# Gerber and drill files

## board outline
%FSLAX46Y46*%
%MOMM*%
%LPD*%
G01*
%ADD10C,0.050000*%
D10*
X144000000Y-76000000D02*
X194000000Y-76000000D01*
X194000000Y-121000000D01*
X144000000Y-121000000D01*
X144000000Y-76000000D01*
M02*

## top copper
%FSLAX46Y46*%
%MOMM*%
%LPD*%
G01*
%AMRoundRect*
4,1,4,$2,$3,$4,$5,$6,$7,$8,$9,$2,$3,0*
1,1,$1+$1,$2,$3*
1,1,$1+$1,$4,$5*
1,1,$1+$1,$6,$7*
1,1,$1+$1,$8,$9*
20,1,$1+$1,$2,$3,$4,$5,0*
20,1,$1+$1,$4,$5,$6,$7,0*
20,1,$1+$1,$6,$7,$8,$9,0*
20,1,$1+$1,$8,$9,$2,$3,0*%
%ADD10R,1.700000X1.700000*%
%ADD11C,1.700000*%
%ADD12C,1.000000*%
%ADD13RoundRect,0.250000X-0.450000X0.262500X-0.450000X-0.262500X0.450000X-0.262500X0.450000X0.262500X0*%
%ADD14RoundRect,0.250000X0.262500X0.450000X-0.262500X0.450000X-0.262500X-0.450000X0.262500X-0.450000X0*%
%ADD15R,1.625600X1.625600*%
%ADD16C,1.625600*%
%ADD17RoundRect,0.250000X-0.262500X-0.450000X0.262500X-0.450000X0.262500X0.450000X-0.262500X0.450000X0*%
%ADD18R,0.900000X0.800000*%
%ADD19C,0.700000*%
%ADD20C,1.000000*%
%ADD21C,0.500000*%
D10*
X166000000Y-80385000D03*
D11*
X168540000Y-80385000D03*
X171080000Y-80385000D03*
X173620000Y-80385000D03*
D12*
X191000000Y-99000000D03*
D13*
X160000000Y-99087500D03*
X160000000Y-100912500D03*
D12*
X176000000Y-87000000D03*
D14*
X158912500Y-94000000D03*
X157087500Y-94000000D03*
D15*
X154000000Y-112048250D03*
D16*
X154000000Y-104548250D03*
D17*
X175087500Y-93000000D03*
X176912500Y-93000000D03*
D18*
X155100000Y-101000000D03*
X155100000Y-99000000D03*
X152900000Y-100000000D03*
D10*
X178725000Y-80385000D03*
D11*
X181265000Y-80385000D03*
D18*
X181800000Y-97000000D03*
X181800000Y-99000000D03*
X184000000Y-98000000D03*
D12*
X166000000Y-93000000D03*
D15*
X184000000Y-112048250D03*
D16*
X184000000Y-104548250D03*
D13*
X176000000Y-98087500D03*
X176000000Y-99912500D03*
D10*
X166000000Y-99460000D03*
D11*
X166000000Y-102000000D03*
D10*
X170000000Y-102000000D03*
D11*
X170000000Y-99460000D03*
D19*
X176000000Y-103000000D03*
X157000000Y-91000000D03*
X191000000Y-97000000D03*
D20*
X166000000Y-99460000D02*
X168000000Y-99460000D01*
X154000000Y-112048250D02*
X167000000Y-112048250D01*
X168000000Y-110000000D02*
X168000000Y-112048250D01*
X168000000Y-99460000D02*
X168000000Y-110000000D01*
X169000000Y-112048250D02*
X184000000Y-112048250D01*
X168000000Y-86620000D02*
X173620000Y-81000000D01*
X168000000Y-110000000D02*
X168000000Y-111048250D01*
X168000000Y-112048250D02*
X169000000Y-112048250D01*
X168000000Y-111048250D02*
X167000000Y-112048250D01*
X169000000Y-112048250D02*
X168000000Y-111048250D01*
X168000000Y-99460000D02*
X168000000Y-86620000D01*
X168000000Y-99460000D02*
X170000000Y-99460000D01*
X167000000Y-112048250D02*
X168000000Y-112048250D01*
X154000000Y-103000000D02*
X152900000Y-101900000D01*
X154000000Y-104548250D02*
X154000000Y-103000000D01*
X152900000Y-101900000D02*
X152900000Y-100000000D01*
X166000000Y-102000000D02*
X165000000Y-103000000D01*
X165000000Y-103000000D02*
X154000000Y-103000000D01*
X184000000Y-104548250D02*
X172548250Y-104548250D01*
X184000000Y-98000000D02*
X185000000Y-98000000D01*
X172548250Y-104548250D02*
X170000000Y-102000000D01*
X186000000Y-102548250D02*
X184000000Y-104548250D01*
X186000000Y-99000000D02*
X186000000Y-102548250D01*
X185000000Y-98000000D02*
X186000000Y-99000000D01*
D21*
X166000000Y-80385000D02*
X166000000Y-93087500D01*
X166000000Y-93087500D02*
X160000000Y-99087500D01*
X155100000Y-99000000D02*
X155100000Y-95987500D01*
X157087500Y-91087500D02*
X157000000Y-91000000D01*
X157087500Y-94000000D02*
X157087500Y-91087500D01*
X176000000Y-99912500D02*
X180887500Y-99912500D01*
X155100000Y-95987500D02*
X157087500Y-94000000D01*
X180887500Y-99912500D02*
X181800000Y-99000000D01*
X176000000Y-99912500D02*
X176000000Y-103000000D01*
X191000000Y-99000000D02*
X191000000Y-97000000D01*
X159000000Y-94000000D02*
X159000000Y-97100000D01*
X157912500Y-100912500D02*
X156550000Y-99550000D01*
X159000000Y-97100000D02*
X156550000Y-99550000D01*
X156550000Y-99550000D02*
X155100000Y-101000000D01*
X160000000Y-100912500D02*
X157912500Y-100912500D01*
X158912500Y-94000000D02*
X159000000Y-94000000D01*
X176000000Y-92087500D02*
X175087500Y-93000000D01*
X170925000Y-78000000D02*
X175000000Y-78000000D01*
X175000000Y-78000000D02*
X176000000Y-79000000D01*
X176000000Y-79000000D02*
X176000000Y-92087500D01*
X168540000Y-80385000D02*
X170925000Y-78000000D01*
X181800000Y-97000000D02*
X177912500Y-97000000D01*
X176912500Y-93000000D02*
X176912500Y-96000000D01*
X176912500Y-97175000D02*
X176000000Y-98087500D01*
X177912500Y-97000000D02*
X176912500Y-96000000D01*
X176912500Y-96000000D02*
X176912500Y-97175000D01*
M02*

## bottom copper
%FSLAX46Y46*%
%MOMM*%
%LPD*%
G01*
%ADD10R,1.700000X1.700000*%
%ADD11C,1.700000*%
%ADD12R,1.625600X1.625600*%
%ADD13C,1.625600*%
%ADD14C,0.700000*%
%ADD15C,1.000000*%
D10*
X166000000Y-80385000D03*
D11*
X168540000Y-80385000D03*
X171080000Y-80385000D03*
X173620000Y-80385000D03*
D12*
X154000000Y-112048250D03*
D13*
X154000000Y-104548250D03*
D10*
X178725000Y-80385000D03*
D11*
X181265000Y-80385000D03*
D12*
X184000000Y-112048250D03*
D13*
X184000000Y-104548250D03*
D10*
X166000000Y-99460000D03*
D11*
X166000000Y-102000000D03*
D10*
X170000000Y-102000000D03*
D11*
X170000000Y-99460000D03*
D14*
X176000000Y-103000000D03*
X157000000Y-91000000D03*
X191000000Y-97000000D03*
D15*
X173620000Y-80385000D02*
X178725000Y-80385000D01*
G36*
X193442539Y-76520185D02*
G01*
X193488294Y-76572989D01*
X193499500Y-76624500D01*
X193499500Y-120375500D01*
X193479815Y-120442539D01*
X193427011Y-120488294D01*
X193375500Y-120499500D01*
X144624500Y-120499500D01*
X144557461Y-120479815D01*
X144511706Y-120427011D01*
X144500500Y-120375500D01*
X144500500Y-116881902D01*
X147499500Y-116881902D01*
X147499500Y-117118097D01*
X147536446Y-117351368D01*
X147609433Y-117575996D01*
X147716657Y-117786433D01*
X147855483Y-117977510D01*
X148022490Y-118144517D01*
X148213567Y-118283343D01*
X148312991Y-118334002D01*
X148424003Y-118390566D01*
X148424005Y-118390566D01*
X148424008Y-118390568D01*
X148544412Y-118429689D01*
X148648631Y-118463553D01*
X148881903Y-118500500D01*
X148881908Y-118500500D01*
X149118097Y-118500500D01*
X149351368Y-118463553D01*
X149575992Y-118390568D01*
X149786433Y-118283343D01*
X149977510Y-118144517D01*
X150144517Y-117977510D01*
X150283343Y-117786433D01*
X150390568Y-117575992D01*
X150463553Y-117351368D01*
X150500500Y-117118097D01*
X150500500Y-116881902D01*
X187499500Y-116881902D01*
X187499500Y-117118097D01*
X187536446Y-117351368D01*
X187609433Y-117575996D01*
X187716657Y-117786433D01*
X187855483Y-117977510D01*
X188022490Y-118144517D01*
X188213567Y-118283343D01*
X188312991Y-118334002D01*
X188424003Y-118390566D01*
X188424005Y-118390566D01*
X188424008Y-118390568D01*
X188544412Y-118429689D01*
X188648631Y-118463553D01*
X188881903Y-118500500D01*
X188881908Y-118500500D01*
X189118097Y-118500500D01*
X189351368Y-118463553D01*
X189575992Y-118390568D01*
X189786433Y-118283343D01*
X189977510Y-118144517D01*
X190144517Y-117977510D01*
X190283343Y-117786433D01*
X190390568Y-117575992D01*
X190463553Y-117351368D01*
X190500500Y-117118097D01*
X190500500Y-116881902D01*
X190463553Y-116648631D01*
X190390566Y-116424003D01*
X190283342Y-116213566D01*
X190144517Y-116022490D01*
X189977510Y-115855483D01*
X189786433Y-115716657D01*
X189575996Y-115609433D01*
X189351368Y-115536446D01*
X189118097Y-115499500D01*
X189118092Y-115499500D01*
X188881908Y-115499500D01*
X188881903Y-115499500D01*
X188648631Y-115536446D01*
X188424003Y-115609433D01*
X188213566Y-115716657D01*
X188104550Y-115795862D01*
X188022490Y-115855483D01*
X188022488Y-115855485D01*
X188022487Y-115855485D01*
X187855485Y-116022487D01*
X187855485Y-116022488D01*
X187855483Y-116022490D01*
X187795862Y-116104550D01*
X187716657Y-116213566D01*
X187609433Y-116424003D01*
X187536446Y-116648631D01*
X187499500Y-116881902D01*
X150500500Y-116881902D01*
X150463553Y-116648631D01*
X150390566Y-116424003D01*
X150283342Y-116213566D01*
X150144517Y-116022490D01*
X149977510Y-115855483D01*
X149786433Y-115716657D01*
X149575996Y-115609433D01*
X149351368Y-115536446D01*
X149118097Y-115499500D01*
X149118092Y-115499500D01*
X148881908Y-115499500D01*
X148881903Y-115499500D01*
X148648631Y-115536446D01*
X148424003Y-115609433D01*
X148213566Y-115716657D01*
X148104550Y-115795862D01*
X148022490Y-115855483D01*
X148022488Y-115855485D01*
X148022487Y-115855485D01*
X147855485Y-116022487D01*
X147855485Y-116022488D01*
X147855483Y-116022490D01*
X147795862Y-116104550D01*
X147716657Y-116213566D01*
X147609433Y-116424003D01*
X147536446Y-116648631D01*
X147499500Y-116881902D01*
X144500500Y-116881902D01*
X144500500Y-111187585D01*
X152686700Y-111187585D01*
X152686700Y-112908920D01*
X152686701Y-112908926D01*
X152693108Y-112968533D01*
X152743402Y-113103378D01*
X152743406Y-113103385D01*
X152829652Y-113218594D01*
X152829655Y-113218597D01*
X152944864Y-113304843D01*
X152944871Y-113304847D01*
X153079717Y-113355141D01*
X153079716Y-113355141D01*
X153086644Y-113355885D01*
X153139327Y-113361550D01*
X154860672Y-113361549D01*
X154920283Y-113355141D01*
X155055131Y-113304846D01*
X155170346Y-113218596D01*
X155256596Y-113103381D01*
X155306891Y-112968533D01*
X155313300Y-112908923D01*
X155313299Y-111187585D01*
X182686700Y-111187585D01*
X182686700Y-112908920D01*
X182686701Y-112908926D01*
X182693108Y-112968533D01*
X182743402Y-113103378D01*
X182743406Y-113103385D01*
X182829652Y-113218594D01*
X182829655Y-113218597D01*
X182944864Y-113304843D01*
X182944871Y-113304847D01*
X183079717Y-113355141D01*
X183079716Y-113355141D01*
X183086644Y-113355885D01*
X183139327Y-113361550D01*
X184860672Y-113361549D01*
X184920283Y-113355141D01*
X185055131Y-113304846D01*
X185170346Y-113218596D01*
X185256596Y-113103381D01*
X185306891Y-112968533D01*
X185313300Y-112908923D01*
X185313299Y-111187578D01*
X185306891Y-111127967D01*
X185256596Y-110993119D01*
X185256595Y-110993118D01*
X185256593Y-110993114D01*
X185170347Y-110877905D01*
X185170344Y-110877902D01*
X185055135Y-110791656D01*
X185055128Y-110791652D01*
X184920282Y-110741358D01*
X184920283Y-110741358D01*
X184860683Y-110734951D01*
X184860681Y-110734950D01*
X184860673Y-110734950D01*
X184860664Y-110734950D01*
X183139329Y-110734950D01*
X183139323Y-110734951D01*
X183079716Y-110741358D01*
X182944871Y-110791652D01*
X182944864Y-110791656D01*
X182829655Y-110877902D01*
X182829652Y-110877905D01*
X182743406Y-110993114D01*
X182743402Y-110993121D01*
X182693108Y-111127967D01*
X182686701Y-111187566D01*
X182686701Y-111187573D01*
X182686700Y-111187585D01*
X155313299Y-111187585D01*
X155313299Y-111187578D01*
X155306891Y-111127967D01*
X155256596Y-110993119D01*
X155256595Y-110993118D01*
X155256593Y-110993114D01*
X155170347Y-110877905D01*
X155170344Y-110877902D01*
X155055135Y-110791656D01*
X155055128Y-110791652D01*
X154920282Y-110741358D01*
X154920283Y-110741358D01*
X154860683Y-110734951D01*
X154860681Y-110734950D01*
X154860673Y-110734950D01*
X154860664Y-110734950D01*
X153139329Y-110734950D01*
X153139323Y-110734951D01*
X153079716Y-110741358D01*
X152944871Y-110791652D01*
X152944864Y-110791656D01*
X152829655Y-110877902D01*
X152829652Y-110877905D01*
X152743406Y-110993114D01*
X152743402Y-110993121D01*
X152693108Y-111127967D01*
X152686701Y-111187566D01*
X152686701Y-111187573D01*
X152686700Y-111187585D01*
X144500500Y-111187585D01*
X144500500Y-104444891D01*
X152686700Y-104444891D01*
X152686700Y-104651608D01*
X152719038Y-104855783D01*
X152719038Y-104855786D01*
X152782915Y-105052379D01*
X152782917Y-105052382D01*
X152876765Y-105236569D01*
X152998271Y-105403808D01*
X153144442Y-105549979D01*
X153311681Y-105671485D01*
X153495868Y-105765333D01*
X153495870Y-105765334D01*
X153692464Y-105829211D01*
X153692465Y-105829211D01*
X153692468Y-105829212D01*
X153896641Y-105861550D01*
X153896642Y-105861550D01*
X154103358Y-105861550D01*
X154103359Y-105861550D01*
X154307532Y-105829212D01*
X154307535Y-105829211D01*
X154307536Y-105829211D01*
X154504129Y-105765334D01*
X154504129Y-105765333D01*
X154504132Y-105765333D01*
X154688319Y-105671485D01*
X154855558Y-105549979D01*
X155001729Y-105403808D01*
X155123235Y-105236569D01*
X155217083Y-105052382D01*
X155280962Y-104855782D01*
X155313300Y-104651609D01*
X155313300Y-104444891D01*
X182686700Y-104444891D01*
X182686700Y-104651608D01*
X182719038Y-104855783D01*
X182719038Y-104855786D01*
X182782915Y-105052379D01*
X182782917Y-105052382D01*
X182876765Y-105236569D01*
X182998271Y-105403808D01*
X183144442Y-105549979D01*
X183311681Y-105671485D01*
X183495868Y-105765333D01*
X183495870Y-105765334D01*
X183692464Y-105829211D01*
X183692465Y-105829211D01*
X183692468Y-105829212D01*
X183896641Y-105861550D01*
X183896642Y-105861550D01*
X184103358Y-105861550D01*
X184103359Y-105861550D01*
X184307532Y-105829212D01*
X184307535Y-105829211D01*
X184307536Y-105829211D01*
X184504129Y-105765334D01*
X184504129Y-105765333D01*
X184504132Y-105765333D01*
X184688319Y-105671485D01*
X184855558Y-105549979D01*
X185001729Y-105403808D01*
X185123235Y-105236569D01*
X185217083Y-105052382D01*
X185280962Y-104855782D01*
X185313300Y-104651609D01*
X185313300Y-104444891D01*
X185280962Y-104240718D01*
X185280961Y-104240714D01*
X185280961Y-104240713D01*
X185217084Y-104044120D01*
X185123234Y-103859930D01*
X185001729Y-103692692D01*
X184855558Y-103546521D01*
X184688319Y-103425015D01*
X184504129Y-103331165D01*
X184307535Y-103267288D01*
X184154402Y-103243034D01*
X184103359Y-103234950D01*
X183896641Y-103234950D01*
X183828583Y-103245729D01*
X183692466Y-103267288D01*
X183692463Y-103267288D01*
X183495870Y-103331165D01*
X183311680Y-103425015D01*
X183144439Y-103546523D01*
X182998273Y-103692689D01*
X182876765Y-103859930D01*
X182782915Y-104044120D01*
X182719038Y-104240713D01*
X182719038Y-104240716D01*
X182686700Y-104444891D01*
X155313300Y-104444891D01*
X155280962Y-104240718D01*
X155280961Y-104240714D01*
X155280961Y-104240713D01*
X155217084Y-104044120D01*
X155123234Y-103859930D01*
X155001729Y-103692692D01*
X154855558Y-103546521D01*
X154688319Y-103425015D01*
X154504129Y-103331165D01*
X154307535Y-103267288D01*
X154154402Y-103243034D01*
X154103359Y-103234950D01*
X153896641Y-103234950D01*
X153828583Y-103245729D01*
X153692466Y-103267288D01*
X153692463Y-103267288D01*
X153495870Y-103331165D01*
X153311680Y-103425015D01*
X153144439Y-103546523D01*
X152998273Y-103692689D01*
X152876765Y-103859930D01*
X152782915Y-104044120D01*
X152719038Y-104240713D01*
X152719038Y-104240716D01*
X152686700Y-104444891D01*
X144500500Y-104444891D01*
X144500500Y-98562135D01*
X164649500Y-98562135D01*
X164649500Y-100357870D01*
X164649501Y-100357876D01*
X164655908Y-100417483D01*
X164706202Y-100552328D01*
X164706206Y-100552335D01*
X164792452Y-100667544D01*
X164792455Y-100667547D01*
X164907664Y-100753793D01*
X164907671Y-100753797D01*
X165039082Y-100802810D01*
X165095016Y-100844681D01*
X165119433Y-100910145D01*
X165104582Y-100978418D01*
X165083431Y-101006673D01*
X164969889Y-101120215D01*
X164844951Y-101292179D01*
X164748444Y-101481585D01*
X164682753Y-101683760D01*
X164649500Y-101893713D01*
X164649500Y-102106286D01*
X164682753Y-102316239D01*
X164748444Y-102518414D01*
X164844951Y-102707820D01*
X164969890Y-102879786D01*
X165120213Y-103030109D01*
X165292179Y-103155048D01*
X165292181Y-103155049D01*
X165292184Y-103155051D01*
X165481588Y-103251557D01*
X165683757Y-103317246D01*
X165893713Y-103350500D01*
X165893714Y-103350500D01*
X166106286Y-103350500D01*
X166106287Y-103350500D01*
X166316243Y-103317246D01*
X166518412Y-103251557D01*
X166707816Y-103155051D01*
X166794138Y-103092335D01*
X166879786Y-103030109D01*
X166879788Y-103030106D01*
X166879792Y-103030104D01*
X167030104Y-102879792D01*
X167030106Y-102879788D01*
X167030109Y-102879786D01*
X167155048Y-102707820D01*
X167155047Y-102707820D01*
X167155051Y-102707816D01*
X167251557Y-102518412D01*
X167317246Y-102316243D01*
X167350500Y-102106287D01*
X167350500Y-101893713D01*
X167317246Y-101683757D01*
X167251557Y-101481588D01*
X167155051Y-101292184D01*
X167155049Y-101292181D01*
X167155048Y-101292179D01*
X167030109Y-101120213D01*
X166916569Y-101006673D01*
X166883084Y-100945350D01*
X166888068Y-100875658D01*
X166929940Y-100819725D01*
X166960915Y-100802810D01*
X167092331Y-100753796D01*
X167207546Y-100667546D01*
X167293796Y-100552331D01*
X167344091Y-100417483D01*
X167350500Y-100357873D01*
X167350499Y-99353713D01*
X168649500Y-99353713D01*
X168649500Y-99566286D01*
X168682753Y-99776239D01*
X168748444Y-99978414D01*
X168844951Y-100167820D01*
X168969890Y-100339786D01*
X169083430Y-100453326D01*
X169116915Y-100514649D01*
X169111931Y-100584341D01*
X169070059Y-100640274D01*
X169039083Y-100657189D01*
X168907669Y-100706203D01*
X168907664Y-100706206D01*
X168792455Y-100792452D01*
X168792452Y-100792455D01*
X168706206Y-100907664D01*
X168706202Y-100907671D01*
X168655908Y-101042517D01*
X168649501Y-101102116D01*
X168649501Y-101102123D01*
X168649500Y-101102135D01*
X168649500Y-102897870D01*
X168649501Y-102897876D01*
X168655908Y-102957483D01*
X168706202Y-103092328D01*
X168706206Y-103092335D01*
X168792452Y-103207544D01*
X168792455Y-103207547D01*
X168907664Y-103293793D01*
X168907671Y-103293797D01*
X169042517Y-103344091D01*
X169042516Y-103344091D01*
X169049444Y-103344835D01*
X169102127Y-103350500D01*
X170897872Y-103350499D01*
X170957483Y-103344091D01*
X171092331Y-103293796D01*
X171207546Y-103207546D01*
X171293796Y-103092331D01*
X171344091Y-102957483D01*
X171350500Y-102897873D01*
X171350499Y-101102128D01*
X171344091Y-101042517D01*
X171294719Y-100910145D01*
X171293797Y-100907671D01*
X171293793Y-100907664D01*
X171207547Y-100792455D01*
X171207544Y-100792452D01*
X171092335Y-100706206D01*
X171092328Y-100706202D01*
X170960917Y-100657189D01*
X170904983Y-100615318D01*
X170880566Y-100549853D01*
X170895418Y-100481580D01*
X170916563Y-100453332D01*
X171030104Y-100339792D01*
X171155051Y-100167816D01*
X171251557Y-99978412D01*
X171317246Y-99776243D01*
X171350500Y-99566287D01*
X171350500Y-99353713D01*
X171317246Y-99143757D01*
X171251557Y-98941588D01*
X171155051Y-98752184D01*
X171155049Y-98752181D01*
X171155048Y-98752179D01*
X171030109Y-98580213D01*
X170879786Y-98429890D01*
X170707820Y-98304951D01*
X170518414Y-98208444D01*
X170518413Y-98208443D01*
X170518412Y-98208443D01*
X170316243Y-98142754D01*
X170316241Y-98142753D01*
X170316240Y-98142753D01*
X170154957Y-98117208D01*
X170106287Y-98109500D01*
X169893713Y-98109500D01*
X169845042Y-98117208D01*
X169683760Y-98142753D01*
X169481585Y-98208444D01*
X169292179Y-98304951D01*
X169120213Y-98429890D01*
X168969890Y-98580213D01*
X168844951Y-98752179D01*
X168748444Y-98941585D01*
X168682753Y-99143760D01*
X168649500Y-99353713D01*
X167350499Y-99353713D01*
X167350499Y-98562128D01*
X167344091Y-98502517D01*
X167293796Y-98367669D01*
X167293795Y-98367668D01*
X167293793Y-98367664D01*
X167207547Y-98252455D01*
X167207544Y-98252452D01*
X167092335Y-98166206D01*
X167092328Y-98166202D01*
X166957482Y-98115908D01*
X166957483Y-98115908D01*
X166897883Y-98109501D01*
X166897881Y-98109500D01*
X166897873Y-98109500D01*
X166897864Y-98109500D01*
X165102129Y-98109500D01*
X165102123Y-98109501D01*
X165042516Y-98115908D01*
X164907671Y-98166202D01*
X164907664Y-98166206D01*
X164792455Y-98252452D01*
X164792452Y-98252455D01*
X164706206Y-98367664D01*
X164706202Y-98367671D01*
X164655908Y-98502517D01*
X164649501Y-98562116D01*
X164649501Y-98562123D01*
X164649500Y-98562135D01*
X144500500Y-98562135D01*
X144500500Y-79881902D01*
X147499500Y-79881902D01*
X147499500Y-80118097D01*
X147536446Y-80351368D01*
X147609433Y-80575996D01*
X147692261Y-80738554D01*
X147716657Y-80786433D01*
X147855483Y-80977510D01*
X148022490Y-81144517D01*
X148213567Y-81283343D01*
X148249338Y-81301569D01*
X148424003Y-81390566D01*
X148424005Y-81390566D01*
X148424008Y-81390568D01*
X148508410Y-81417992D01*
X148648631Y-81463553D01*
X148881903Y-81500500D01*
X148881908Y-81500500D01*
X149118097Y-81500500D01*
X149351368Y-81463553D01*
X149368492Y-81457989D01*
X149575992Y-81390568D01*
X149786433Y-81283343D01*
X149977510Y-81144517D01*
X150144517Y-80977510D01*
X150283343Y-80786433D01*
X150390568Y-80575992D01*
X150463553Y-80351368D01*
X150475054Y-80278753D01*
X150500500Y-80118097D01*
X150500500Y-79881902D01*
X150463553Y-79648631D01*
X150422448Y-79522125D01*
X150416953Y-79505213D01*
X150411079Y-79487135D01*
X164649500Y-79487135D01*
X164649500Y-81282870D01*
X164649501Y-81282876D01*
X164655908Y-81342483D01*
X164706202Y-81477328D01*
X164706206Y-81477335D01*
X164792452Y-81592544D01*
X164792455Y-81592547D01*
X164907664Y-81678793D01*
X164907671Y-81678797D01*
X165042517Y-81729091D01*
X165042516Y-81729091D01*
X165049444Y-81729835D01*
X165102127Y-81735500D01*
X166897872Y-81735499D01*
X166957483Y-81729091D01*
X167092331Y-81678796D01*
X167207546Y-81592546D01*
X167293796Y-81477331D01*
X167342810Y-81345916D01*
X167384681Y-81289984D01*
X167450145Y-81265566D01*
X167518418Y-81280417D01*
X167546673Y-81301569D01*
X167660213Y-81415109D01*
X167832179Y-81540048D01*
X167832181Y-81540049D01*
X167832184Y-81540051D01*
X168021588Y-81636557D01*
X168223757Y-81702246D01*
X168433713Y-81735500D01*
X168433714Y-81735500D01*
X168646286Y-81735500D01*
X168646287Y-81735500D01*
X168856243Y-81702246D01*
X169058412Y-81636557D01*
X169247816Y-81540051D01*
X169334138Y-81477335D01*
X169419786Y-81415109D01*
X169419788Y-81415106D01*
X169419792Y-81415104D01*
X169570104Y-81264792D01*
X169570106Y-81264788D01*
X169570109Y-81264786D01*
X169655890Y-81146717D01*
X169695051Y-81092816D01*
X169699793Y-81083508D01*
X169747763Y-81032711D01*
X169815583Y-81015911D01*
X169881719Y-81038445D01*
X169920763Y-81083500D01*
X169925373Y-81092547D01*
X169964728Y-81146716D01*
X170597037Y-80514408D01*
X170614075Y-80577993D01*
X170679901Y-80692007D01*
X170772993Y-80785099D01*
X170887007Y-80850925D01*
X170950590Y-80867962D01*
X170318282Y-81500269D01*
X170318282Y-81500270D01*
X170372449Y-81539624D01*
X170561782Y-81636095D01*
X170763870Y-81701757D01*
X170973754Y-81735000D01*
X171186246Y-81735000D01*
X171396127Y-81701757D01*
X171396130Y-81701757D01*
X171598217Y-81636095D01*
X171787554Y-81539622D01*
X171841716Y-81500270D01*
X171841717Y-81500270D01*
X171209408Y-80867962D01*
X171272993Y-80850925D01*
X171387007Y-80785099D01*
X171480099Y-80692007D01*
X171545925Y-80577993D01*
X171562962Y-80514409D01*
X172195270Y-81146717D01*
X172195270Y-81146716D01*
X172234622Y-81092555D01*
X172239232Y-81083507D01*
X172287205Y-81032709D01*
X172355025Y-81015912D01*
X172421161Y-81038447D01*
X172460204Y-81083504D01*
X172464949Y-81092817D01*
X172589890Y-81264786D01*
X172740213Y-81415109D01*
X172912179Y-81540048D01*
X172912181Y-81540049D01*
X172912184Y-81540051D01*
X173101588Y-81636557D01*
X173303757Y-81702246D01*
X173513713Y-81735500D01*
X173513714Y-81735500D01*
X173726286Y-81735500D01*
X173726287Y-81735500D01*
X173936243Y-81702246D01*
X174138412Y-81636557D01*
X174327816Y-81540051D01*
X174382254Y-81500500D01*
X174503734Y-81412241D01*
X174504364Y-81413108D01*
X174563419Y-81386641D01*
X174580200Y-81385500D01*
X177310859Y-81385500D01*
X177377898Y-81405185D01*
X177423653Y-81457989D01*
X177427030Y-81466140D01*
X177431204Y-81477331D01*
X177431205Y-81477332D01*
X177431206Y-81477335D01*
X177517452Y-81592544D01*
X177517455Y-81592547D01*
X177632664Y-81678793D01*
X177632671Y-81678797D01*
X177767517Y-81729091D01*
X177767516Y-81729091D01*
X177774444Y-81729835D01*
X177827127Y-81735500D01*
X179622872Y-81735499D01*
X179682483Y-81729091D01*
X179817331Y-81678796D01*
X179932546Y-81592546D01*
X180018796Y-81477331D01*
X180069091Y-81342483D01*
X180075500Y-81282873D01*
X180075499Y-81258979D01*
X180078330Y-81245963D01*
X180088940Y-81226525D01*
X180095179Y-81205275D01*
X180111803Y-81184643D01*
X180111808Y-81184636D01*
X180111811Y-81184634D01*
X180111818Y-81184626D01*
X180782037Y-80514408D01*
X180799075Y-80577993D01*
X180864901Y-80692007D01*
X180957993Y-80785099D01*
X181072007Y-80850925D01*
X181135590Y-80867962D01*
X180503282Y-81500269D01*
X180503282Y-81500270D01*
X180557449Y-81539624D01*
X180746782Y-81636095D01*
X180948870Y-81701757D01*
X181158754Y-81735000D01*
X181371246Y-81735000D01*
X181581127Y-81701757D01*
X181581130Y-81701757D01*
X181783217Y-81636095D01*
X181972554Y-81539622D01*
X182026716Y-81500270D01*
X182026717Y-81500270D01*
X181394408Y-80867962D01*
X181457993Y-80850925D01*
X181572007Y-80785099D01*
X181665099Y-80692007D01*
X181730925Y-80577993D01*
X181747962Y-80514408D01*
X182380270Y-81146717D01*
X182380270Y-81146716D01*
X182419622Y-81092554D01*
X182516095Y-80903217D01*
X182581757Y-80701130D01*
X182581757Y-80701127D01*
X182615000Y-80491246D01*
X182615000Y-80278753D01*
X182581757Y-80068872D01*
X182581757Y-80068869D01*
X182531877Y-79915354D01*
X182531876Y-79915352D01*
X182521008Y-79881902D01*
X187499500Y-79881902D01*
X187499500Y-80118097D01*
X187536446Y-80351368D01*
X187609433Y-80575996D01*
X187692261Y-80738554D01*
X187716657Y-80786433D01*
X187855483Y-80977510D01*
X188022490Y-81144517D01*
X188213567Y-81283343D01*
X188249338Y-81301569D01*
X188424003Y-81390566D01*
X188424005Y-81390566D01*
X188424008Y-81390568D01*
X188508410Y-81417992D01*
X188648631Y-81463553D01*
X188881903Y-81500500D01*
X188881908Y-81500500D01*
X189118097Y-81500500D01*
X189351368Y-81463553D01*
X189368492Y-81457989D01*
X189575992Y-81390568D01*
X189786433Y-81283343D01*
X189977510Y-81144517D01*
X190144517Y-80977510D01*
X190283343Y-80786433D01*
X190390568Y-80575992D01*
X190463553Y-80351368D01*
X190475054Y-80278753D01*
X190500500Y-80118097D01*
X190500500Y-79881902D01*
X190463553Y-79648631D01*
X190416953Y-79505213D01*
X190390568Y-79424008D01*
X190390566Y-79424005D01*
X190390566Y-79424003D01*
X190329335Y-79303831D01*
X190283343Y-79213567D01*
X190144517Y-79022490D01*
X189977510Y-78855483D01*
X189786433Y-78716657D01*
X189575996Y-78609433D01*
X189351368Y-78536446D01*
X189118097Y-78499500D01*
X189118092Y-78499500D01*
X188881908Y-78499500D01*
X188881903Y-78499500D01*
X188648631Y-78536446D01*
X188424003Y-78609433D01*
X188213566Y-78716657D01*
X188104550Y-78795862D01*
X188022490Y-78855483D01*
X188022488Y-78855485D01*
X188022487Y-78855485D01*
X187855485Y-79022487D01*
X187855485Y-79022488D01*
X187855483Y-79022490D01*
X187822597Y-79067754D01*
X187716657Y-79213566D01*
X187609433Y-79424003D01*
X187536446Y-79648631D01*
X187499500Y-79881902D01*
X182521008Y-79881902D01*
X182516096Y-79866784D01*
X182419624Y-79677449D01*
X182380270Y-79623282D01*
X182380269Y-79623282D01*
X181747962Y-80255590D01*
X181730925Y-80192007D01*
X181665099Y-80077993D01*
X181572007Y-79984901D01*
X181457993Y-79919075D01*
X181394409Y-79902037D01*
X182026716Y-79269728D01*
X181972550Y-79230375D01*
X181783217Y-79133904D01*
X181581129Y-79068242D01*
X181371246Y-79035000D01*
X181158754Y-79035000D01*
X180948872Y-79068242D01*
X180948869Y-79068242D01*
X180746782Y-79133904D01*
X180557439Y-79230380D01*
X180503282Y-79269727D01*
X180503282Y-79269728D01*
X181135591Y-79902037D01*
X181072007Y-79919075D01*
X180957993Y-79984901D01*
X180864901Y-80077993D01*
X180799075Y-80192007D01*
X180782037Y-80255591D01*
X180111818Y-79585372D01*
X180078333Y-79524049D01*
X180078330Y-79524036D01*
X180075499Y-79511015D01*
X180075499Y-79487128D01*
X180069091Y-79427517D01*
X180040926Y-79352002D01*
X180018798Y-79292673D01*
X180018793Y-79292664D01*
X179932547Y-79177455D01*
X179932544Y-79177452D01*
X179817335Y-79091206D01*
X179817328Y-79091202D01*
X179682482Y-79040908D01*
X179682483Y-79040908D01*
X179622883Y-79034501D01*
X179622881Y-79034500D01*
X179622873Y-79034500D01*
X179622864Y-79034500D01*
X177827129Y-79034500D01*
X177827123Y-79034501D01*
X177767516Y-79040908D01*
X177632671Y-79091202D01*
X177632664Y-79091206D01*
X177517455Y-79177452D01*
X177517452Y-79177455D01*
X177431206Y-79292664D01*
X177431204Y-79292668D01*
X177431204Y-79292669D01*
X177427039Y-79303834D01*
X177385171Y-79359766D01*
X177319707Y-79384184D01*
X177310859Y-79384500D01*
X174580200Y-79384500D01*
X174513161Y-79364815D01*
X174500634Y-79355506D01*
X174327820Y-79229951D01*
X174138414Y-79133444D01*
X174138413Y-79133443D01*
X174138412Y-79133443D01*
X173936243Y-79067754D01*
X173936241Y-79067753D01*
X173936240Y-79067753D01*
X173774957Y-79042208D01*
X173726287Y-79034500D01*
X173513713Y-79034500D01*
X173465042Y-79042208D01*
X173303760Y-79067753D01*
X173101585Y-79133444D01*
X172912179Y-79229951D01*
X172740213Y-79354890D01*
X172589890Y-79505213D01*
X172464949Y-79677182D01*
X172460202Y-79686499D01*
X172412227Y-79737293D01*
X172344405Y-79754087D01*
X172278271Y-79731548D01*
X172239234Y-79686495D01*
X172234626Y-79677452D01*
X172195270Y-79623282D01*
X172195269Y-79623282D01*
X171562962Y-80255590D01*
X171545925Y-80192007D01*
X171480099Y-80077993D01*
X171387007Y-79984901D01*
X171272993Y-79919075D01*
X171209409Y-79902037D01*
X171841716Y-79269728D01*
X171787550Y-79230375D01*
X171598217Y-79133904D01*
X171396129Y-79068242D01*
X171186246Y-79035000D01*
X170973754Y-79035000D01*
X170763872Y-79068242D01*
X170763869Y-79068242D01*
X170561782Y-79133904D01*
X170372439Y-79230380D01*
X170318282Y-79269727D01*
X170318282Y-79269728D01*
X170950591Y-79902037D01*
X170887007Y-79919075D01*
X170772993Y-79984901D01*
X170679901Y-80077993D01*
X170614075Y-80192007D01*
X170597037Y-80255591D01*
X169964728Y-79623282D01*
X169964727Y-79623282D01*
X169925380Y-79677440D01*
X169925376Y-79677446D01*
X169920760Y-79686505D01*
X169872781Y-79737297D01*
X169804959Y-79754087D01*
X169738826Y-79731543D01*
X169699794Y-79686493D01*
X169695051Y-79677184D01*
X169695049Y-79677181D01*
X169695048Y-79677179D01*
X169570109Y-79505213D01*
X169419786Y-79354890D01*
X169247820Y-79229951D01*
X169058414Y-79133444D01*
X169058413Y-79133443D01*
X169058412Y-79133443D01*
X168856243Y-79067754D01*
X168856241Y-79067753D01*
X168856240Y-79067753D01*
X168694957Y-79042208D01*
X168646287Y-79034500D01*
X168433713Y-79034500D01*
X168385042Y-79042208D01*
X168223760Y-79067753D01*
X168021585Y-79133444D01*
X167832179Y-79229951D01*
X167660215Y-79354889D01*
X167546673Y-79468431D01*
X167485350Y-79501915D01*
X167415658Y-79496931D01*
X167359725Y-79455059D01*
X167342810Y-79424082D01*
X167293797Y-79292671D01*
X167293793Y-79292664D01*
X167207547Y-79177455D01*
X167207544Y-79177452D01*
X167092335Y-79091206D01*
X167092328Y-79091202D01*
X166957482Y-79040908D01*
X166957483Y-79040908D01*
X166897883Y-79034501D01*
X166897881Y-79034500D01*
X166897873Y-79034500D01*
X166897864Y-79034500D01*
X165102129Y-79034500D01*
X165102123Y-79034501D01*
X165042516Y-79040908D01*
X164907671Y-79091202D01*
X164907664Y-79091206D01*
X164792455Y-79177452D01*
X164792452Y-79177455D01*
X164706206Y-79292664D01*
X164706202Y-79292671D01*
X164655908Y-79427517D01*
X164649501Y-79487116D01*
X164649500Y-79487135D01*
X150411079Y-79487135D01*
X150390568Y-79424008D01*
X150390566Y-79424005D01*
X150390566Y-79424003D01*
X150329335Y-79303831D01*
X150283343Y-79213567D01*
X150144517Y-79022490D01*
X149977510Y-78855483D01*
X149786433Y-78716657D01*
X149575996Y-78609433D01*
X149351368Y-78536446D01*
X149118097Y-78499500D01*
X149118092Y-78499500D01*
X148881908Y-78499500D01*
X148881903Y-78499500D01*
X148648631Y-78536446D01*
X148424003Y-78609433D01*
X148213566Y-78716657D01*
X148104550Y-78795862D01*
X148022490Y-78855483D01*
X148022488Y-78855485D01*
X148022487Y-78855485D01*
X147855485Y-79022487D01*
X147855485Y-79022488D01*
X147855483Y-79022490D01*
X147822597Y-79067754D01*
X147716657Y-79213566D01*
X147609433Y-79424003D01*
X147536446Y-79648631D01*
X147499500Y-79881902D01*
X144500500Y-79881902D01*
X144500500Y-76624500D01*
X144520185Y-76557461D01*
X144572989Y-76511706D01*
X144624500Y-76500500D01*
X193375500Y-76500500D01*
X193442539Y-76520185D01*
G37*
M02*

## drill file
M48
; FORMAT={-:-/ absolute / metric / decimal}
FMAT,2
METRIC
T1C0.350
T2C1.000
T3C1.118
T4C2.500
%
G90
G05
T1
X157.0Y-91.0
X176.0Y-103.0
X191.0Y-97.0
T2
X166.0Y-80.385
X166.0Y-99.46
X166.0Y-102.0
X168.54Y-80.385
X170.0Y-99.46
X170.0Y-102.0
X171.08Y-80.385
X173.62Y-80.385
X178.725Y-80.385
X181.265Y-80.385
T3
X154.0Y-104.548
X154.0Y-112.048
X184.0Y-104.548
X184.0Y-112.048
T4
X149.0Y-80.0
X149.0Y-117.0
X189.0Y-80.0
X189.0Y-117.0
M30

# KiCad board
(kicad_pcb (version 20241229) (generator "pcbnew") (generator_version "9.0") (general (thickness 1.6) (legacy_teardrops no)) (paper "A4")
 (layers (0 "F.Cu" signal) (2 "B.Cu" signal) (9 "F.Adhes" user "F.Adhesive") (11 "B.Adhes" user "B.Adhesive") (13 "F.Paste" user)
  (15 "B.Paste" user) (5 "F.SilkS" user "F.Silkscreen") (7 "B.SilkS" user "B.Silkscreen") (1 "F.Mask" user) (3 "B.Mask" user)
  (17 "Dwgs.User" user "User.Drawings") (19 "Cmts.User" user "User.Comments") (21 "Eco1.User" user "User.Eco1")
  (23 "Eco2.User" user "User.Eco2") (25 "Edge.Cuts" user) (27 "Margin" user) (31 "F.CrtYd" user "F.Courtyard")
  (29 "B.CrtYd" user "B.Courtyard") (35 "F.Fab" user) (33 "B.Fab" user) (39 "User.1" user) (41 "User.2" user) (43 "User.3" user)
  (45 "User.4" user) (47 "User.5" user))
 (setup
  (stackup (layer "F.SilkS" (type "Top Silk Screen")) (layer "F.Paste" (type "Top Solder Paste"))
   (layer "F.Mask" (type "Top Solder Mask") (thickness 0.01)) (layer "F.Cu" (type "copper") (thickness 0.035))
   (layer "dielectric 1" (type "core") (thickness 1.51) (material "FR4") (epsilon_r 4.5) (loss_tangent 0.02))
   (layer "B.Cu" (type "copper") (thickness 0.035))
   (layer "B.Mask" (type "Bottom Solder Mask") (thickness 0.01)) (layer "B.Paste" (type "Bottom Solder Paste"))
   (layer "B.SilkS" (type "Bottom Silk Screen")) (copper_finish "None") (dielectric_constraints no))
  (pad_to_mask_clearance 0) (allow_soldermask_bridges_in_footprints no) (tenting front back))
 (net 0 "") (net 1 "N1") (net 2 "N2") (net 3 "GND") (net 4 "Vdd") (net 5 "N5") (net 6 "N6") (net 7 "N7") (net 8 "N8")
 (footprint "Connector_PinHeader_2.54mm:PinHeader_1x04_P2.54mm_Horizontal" (layer "F.Cu") (at 166 80.385 90)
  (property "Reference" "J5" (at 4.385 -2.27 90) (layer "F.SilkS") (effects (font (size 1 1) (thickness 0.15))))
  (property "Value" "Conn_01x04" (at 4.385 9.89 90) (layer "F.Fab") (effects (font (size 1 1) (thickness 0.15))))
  (pad "1" thru_hole rect (at 0 0 90) (size 1.7 1.7) (drill 1) (layers "*.Cu" "*.Mask") (remove_unused_layers no) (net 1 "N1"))
  (pad "2" thru_hole circle (at 0 2.54 90) (size 1.7 1.7) (drill 1) (layers "*.Cu" "*.Mask") (remove_unused_layers no) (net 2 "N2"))
  (pad "3" thru_hole circle (at 0 5.08 90) (size 1.7 1.7) (drill 1) (layers "*.Cu" "*.Mask") (remove_unused_layers no) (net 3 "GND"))
  (pad "4" thru_hole circle (at 0 7.62 90) (size 1.7 1.7) (drill 1) (layers "*.Cu" "*.Mask") (remove_unused_layers no) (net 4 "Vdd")))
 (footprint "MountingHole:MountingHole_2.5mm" (layer "F.Cu") (at 189 80)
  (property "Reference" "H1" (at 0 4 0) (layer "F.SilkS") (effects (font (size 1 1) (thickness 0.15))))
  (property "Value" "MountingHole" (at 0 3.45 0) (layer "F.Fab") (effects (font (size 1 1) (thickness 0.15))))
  (pad "" np_thru_hole circle (at 0 0) (size 2.5 2.5) (drill 2.5) (layers "*.Cu" "*.Mask")))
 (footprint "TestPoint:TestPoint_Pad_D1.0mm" (layer "F.Cu") (at 191 99)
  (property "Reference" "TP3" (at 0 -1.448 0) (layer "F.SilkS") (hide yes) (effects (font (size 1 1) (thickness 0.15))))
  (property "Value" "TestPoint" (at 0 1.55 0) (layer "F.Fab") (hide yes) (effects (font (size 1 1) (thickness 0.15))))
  (pad "1" smd circle (at 0 0) (size 1 1) (layers "F.Cu" "F.Mask") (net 3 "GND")))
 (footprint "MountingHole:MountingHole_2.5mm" (layer "F.Cu") (at 189 117)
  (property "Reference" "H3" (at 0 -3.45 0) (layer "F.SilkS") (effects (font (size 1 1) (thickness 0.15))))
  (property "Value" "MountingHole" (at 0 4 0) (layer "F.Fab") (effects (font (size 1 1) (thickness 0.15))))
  (pad "" np_thru_hole circle (at 0 0) (size 2.5 2.5) (drill 2.5) (layers "*.Cu" "*.Mask")))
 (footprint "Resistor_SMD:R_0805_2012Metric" (layer "F.Cu") (at 160 100 -90)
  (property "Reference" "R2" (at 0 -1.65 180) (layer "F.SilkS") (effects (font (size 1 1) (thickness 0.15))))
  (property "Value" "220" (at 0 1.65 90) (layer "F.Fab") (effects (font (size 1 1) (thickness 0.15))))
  (pad "1" smd roundrect (at -0.9125 0 270) (size 1.025 1.4) (layers "F.Cu" "F.Mask" "F.Paste") (roundrect_rratio 0.243902) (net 1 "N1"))
  (pad "2" smd roundrect (at 0.9125 0 270) (size 1.025 1.4) (layers "F.Cu" "F.Mask" "F.Paste") (roundrect_rratio 0.243902) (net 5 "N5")))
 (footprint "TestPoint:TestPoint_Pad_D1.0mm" (layer "F.Cu") (at 176 87)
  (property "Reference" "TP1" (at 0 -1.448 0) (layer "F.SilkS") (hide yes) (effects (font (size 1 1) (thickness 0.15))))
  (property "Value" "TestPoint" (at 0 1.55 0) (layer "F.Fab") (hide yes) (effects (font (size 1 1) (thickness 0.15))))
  (pad "1" smd circle (at 0 0) (size 1 1) (layers "F.Cu" "F.Mask") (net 2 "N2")))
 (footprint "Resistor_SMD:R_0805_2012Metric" (layer "F.Cu") (at 158 94 180)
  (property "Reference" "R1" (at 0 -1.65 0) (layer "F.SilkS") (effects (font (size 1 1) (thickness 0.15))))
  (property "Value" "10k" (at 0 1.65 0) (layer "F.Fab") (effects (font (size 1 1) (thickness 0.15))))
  (pad "1" smd roundrect (at -0.9125 0 180) (size 1.025 1.4) (layers "F.Cu" "F.Mask" "F.Paste") (roundrect_rratio 0.243902) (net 5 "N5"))
  (pad "2" smd roundrect (at 0.9125 0 180) (size 1.025 1.4) (layers "F.Cu" "F.Mask" "F.Paste") (roundrect_rratio 0.243902) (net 3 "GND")))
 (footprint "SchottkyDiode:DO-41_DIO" (layer "F.Cu") (at 154 114.04825 90)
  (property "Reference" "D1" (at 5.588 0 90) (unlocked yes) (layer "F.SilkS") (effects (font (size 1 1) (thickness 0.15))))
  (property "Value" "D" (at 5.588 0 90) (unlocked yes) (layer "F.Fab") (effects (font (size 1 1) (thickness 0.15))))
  (pad "1" thru_hole rect (at 2 0 90) (size 1.6256 1.6256) (drill 1.1176) (layers "*.Cu" "*.Mask") (remove_unused_layers no) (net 4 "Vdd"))
  (pad "2" thru_hole circle (at 9.5 0 90) (size 1.6256 1.6256) (drill 1.1176) (layers "*.Cu" "*.Mask") (remove_unused_layers no)
   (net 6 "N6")))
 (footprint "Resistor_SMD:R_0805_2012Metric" (layer "F.Cu") (at 176 93)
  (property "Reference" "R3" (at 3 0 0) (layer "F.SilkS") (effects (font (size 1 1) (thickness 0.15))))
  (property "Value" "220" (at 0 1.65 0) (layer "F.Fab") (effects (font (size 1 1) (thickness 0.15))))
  (pad "1" smd roundrect (at -0.9125 0) (size 1.025 1.4) (layers "F.Cu" "F.Mask" "F.Paste") (roundrect_rratio 0.243902) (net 2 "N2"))
  (pad "2" smd roundrect (at 0.9125 0) (size 1.025 1.4) (layers "F.Cu" "F.Mask" "F.Paste") (roundrect_rratio 0.243902) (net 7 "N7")))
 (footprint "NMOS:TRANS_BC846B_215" (layer "F.Cu") (at 154 100 90)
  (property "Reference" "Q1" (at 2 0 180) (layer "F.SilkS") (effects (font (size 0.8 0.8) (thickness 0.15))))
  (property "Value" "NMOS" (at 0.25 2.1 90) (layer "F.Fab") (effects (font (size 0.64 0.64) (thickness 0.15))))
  (pad "1" smd rect (at -1 1.1 90) (size 0.8 0.9) (layers "F.Cu" "F.Mask" "F.Paste") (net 5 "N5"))
  (pad "2" smd rect (at 1 1.1 90) (size 0.8 0.9) (layers "F.Cu" "F.Mask" "F.Paste") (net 3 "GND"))
  (pad "3" smd rect (at 0 -1.1 90) (size 0.8 0.9) (layers "F.Cu" "F.Mask" "F.Paste") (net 6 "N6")))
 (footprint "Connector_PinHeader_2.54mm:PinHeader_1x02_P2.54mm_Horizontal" (layer "F.Cu") (at 178.725 80.385 90)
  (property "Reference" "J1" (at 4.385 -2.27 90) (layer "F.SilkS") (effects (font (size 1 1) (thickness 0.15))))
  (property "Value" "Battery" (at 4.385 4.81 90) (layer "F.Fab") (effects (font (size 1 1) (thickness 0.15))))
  (pad "1" thru_hole rect (at 0 0 90) (size 1.7 1.7) (drill 1) (layers "*.Cu" "*.Mask") (remove_unused_layers no) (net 4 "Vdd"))
  (pad "2" thru_hole circle (at 0 2.54 90) (size 1.7 1.7) (drill 1) (layers "*.Cu" "*.Mask") (remove_unused_layers no) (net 3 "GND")))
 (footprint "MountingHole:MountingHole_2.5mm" (layer "F.Cu") (at 149 80)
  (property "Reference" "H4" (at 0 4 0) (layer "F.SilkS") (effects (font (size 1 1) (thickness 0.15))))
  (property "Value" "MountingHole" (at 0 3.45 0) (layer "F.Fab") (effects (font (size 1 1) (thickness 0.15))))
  (pad "" np_thru_hole circle (at 0 0) (size 2.5 2.5) (drill 2.5) (layers "*.Cu" "*.Mask")))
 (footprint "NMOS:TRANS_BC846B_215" (layer "F.Cu") (at 182.9 98 -90)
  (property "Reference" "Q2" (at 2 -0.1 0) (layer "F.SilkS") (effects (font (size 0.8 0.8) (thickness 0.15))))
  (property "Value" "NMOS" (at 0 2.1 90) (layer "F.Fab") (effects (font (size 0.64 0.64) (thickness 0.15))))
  (pad "1" smd rect (at -1 1.1 270) (size 0.8 0.9) (layers "F.Cu" "F.Mask" "F.Paste") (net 7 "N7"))
  (pad "2" smd rect (at 1 1.1 270) (size 0.8 0.9) (layers "F.Cu" "F.Mask" "F.Paste") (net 3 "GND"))
  (pad "3" smd rect (at 0 -1.1 270) (size 0.8 0.9) (layers "F.Cu" "F.Mask" "F.Paste") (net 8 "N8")))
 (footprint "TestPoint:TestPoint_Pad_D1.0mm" (layer "F.Cu") (at 166 93)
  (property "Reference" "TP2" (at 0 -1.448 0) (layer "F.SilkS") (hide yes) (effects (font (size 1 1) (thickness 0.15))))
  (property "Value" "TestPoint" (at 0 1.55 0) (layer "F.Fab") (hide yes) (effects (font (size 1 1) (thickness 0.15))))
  (pad "1" smd circle (at 0 0) (size 1 1) (layers "F.Cu" "F.Mask") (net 1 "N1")))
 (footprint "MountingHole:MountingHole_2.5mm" (layer "F.Cu") (at 149 117)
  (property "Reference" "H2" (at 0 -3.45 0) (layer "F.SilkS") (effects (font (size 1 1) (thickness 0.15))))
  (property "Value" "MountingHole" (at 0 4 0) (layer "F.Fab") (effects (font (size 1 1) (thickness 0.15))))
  (pad "" np_thru_hole circle (at 0 0) (size 2.5 2.5) (drill 2.5) (layers "*.Cu" "*.Mask")))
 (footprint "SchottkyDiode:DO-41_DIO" (layer "F.Cu") (at 184 114.04825 90)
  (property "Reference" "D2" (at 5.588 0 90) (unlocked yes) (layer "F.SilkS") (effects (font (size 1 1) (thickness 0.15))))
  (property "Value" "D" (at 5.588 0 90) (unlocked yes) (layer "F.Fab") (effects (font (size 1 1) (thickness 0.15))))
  (pad "1" thru_hole rect (at 2 0 90) (size 1.6256 1.6256) (drill 1.1176) (layers "*.Cu" "*.Mask") (remove_unused_layers no) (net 4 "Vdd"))
  (pad "2" thru_hole circle (at 9.5 0 90) (size 1.6256 1.6256) (drill 1.1176) (layers "*.Cu" "*.Mask") (remove_unused_layers no)
   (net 8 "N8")))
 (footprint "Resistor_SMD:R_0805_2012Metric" (layer "F.Cu") (at 176 99 -90)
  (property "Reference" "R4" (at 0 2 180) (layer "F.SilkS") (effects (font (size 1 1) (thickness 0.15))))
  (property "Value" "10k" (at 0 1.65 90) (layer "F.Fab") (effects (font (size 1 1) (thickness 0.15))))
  (pad "1" smd roundrect (at -0.9125 0 270) (size 1.025 1.4) (layers "F.Cu" "F.Mask" "F.Paste") (roundrect_rratio 0.243902) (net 7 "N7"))
  (pad "2" smd roundrect (at 0.9125 0 270) (size 1.025 1.4) (layers "F.Cu" "F.Mask" "F.Paste") (roundrect_rratio 0.243902) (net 3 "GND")))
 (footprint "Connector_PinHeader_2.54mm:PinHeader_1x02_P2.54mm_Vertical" (layer "B.Cu") (at 166 99.46 180)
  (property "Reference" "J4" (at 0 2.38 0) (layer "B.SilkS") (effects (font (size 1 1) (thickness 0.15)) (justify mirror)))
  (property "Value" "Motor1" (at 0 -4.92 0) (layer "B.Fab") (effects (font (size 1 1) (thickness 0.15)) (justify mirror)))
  (pad "1" thru_hole rect (at 0 0 180) (size 1.7 1.7) (drill 1) (layers "*.Cu" "*.Mask") (remove_unused_layers no) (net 4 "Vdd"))
  (pad "2" thru_hole circle (at 0 -2.54 180) (size 1.7 1.7) (drill 1) (layers "*.Cu" "*.Mask") (remove_unused_layers no) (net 6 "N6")))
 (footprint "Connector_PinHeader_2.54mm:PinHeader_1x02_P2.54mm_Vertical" (layer "B.Cu") (at 170 102)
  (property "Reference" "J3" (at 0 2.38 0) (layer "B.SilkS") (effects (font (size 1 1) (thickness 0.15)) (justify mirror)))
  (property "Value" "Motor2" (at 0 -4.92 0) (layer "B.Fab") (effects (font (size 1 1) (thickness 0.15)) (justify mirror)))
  (pad "1" thru_hole rect (at 0 0) (size 1.7 1.7) (drill 1) (layers "*.Cu" "*.Mask") (remove_unused_layers no) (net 8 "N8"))
  (pad "2" thru_hole circle (at 0 -2.54) (size 1.7 1.7) (drill 1) (layers "*.Cu" "*.Mask") (remove_unused_layers no) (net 4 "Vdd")))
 (gr_rect (start 144 76) (end 194 121) (stroke (width 0.05) (type default)) (fill no) (layer "Edge.Cuts"))
 (segment (start 166 99.46) (end 168 99.46) (width 1) (layer "F.Cu") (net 4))
 (segment (start 154 112.04825) (end 167 112.04825) (width 1) (layer "F.Cu") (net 4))
 (segment (start 168 110) (end 168 112.04825) (width 1) (layer "F.Cu") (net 4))
 (segment (start 168 99.46) (end 168 110) (width 1) (layer "F.Cu") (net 4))
 (segment (start 169 112.04825) (end 184 112.04825) (width 1) (layer "F.Cu") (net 4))
 (segment (start 168 86.62) (end 173.62 81) (width 1) (layer "F.Cu") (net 4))
 (segment (start 168 110) (end 168 111.04825) (width 1) (layer "F.Cu") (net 4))
 (segment (start 168 112.04825) (end 169 112.04825) (width 1) (layer "F.Cu") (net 4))
 (segment (start 168 111.04825) (end 167 112.04825) (width 1) (layer "F.Cu") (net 4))
 (segment (start 169 112.04825) (end 168 111.04825) (width 1) (layer "F.Cu") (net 4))
 (segment (start 168 99.46) (end 168 86.62) (width 1) (layer "F.Cu") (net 4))
 (segment (start 168 99.46) (end 170 99.46) (width 1) (layer "F.Cu") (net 4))
 (segment (start 167 112.04825) (end 168 112.04825) (width 1) (layer "F.Cu") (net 4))
 (segment (start 173.62 80.385) (end 178.725 80.385) (width 1) (layer "B.Cu") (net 4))
 (segment (start 154 103) (end 152.9 101.9) (width 1) (layer "F.Cu") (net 6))
 (segment (start 154 104.54825) (end 154 103) (width 1) (layer "F.Cu") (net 6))
 (segment (start 152.9 101.9) (end 152.9 100) (width 1) (layer "F.Cu") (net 6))
 (segment (start 166 102) (end 165 103) (width 1) (layer "F.Cu") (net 6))
 (segment (start 165 103) (end 154 103) (width 1) (layer "F.Cu") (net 6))
 (segment (start 184 104.54825) (end 172.54825 104.54825) (width 1) (layer "F.Cu") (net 8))
 (segment (start 184 98) (end 185 98) (width 1) (layer "F.Cu") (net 8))
 (segment (start 172.54825 104.54825) (end 170 102) (width 1) (layer "F.Cu") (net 8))
 (segment (start 186 102.54825) (end 184 104.54825) (width 1) (layer "F.Cu") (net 8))
 (segment (start 186 99) (end 186 102.54825) (width 1) (layer "F.Cu") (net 8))
 (segment (start 185 98) (end 186 99) (width 1) (layer "F.Cu") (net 8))
 (segment (start 166 80.385) (end 166 93.0875) (width 0.5) (layer "F.Cu") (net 1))
 (segment (start 166 93.0875) (end 160 99.0875) (width 0.5) (layer "F.Cu") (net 1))
 (segment (start 155.1 99) (end 155.1 95.9875) (width 0.5) (layer "F.Cu") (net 3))
 (segment (start 157.0875 91.0875) (end 157 91) (width 0.5) (layer "F.Cu") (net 3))
 (segment (start 157.0875 94) (end 157.0875 91.0875) (width 0.5) (layer "F.Cu") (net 3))
 (segment (start 176 99.9125) (end 180.8875 99.9125) (width 0.5) (layer "F.Cu") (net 3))
 (segment (start 155.1 95.9875) (end 157.0875 94) (width 0.5) (layer "F.Cu") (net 3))
 (segment (start 180.8875 99.9125) (end 181.8 99) (width 0.5) (layer "F.Cu") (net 3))
 (segment (start 176 99.9125) (end 176 103) (width 0.5) (layer "F.Cu") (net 3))
 (segment (start 191 99) (end 191 97) (width 0.5) (layer "F.Cu") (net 3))
 (via (at 176 103) (size 0.7) (drill 0.35) (layers "F.Cu" "B.Cu") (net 3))
 (via (at 157 91) (size 0.7) (drill 0.35) (layers "F.Cu" "B.Cu") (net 3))
 (via (at 191 97) (size 0.7) (drill 0.35) (layers "F.Cu" "B.Cu") (free yes) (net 3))
 (segment (start 159 94) (end 159 97.1) (width 0.5) (layer "F.Cu") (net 5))
 (segment (start 157.9125 100.9125) (end 156.55 99.55) (width 0.5) (layer "F.Cu") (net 5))
 (segment (start 159 97.1) (end 156.55 99.55) (width 0.5) (layer "F.Cu") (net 5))
 (segment (start 156.55 99.55) (end 155.1 101) (width 0.5) (layer "F.Cu") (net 5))
 (segment (start 160 100.9125) (end 157.9125 100.9125) (width 0.5) (layer "F.Cu") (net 5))
 (segment (start 158.9125 94) (end 159 94) (width 0.5) (layer "F.Cu") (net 5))
 (segment (start 176 92.0875) (end 175.0875 93) (width 0.5) (layer "F.Cu") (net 2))
 (segment (start 170.925 78) (end 175 78) (width 0.5) (layer "F.Cu") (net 2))
 (segment (start 175 78) (end 176 79) (width 0.5) (layer "F.Cu") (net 2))
 (segment (start 176 79) (end 176 92.0875) (width 0.5) (layer "F.Cu") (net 2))
 (segment (start 168.54 80.385) (end 170.925 78) (width 0.5) (layer "F.Cu") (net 2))
 (segment (start 181.8 97) (end 177.9125 97) (width 0.5) (layer "F.Cu") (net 7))
 (segment (start 176.9125 93) (end 176.9125 96) (width 0.5) (layer "F.Cu") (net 7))
 (segment (start 176.9125 97.175) (end 176 98.0875) (width 0.5) (layer "F.Cu") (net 7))
 (segment (start 177.9125 97) (end 176.9125 96) (width 0.5) (layer "F.Cu") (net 7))
 (segment (start 176.9125 96) (end 176.9125 97.175) (width 0.5) (layer "F.Cu") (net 7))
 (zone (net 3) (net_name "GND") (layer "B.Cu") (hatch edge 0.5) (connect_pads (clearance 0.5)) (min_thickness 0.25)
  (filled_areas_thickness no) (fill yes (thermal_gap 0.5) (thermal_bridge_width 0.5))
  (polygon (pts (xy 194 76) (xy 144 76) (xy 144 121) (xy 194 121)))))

